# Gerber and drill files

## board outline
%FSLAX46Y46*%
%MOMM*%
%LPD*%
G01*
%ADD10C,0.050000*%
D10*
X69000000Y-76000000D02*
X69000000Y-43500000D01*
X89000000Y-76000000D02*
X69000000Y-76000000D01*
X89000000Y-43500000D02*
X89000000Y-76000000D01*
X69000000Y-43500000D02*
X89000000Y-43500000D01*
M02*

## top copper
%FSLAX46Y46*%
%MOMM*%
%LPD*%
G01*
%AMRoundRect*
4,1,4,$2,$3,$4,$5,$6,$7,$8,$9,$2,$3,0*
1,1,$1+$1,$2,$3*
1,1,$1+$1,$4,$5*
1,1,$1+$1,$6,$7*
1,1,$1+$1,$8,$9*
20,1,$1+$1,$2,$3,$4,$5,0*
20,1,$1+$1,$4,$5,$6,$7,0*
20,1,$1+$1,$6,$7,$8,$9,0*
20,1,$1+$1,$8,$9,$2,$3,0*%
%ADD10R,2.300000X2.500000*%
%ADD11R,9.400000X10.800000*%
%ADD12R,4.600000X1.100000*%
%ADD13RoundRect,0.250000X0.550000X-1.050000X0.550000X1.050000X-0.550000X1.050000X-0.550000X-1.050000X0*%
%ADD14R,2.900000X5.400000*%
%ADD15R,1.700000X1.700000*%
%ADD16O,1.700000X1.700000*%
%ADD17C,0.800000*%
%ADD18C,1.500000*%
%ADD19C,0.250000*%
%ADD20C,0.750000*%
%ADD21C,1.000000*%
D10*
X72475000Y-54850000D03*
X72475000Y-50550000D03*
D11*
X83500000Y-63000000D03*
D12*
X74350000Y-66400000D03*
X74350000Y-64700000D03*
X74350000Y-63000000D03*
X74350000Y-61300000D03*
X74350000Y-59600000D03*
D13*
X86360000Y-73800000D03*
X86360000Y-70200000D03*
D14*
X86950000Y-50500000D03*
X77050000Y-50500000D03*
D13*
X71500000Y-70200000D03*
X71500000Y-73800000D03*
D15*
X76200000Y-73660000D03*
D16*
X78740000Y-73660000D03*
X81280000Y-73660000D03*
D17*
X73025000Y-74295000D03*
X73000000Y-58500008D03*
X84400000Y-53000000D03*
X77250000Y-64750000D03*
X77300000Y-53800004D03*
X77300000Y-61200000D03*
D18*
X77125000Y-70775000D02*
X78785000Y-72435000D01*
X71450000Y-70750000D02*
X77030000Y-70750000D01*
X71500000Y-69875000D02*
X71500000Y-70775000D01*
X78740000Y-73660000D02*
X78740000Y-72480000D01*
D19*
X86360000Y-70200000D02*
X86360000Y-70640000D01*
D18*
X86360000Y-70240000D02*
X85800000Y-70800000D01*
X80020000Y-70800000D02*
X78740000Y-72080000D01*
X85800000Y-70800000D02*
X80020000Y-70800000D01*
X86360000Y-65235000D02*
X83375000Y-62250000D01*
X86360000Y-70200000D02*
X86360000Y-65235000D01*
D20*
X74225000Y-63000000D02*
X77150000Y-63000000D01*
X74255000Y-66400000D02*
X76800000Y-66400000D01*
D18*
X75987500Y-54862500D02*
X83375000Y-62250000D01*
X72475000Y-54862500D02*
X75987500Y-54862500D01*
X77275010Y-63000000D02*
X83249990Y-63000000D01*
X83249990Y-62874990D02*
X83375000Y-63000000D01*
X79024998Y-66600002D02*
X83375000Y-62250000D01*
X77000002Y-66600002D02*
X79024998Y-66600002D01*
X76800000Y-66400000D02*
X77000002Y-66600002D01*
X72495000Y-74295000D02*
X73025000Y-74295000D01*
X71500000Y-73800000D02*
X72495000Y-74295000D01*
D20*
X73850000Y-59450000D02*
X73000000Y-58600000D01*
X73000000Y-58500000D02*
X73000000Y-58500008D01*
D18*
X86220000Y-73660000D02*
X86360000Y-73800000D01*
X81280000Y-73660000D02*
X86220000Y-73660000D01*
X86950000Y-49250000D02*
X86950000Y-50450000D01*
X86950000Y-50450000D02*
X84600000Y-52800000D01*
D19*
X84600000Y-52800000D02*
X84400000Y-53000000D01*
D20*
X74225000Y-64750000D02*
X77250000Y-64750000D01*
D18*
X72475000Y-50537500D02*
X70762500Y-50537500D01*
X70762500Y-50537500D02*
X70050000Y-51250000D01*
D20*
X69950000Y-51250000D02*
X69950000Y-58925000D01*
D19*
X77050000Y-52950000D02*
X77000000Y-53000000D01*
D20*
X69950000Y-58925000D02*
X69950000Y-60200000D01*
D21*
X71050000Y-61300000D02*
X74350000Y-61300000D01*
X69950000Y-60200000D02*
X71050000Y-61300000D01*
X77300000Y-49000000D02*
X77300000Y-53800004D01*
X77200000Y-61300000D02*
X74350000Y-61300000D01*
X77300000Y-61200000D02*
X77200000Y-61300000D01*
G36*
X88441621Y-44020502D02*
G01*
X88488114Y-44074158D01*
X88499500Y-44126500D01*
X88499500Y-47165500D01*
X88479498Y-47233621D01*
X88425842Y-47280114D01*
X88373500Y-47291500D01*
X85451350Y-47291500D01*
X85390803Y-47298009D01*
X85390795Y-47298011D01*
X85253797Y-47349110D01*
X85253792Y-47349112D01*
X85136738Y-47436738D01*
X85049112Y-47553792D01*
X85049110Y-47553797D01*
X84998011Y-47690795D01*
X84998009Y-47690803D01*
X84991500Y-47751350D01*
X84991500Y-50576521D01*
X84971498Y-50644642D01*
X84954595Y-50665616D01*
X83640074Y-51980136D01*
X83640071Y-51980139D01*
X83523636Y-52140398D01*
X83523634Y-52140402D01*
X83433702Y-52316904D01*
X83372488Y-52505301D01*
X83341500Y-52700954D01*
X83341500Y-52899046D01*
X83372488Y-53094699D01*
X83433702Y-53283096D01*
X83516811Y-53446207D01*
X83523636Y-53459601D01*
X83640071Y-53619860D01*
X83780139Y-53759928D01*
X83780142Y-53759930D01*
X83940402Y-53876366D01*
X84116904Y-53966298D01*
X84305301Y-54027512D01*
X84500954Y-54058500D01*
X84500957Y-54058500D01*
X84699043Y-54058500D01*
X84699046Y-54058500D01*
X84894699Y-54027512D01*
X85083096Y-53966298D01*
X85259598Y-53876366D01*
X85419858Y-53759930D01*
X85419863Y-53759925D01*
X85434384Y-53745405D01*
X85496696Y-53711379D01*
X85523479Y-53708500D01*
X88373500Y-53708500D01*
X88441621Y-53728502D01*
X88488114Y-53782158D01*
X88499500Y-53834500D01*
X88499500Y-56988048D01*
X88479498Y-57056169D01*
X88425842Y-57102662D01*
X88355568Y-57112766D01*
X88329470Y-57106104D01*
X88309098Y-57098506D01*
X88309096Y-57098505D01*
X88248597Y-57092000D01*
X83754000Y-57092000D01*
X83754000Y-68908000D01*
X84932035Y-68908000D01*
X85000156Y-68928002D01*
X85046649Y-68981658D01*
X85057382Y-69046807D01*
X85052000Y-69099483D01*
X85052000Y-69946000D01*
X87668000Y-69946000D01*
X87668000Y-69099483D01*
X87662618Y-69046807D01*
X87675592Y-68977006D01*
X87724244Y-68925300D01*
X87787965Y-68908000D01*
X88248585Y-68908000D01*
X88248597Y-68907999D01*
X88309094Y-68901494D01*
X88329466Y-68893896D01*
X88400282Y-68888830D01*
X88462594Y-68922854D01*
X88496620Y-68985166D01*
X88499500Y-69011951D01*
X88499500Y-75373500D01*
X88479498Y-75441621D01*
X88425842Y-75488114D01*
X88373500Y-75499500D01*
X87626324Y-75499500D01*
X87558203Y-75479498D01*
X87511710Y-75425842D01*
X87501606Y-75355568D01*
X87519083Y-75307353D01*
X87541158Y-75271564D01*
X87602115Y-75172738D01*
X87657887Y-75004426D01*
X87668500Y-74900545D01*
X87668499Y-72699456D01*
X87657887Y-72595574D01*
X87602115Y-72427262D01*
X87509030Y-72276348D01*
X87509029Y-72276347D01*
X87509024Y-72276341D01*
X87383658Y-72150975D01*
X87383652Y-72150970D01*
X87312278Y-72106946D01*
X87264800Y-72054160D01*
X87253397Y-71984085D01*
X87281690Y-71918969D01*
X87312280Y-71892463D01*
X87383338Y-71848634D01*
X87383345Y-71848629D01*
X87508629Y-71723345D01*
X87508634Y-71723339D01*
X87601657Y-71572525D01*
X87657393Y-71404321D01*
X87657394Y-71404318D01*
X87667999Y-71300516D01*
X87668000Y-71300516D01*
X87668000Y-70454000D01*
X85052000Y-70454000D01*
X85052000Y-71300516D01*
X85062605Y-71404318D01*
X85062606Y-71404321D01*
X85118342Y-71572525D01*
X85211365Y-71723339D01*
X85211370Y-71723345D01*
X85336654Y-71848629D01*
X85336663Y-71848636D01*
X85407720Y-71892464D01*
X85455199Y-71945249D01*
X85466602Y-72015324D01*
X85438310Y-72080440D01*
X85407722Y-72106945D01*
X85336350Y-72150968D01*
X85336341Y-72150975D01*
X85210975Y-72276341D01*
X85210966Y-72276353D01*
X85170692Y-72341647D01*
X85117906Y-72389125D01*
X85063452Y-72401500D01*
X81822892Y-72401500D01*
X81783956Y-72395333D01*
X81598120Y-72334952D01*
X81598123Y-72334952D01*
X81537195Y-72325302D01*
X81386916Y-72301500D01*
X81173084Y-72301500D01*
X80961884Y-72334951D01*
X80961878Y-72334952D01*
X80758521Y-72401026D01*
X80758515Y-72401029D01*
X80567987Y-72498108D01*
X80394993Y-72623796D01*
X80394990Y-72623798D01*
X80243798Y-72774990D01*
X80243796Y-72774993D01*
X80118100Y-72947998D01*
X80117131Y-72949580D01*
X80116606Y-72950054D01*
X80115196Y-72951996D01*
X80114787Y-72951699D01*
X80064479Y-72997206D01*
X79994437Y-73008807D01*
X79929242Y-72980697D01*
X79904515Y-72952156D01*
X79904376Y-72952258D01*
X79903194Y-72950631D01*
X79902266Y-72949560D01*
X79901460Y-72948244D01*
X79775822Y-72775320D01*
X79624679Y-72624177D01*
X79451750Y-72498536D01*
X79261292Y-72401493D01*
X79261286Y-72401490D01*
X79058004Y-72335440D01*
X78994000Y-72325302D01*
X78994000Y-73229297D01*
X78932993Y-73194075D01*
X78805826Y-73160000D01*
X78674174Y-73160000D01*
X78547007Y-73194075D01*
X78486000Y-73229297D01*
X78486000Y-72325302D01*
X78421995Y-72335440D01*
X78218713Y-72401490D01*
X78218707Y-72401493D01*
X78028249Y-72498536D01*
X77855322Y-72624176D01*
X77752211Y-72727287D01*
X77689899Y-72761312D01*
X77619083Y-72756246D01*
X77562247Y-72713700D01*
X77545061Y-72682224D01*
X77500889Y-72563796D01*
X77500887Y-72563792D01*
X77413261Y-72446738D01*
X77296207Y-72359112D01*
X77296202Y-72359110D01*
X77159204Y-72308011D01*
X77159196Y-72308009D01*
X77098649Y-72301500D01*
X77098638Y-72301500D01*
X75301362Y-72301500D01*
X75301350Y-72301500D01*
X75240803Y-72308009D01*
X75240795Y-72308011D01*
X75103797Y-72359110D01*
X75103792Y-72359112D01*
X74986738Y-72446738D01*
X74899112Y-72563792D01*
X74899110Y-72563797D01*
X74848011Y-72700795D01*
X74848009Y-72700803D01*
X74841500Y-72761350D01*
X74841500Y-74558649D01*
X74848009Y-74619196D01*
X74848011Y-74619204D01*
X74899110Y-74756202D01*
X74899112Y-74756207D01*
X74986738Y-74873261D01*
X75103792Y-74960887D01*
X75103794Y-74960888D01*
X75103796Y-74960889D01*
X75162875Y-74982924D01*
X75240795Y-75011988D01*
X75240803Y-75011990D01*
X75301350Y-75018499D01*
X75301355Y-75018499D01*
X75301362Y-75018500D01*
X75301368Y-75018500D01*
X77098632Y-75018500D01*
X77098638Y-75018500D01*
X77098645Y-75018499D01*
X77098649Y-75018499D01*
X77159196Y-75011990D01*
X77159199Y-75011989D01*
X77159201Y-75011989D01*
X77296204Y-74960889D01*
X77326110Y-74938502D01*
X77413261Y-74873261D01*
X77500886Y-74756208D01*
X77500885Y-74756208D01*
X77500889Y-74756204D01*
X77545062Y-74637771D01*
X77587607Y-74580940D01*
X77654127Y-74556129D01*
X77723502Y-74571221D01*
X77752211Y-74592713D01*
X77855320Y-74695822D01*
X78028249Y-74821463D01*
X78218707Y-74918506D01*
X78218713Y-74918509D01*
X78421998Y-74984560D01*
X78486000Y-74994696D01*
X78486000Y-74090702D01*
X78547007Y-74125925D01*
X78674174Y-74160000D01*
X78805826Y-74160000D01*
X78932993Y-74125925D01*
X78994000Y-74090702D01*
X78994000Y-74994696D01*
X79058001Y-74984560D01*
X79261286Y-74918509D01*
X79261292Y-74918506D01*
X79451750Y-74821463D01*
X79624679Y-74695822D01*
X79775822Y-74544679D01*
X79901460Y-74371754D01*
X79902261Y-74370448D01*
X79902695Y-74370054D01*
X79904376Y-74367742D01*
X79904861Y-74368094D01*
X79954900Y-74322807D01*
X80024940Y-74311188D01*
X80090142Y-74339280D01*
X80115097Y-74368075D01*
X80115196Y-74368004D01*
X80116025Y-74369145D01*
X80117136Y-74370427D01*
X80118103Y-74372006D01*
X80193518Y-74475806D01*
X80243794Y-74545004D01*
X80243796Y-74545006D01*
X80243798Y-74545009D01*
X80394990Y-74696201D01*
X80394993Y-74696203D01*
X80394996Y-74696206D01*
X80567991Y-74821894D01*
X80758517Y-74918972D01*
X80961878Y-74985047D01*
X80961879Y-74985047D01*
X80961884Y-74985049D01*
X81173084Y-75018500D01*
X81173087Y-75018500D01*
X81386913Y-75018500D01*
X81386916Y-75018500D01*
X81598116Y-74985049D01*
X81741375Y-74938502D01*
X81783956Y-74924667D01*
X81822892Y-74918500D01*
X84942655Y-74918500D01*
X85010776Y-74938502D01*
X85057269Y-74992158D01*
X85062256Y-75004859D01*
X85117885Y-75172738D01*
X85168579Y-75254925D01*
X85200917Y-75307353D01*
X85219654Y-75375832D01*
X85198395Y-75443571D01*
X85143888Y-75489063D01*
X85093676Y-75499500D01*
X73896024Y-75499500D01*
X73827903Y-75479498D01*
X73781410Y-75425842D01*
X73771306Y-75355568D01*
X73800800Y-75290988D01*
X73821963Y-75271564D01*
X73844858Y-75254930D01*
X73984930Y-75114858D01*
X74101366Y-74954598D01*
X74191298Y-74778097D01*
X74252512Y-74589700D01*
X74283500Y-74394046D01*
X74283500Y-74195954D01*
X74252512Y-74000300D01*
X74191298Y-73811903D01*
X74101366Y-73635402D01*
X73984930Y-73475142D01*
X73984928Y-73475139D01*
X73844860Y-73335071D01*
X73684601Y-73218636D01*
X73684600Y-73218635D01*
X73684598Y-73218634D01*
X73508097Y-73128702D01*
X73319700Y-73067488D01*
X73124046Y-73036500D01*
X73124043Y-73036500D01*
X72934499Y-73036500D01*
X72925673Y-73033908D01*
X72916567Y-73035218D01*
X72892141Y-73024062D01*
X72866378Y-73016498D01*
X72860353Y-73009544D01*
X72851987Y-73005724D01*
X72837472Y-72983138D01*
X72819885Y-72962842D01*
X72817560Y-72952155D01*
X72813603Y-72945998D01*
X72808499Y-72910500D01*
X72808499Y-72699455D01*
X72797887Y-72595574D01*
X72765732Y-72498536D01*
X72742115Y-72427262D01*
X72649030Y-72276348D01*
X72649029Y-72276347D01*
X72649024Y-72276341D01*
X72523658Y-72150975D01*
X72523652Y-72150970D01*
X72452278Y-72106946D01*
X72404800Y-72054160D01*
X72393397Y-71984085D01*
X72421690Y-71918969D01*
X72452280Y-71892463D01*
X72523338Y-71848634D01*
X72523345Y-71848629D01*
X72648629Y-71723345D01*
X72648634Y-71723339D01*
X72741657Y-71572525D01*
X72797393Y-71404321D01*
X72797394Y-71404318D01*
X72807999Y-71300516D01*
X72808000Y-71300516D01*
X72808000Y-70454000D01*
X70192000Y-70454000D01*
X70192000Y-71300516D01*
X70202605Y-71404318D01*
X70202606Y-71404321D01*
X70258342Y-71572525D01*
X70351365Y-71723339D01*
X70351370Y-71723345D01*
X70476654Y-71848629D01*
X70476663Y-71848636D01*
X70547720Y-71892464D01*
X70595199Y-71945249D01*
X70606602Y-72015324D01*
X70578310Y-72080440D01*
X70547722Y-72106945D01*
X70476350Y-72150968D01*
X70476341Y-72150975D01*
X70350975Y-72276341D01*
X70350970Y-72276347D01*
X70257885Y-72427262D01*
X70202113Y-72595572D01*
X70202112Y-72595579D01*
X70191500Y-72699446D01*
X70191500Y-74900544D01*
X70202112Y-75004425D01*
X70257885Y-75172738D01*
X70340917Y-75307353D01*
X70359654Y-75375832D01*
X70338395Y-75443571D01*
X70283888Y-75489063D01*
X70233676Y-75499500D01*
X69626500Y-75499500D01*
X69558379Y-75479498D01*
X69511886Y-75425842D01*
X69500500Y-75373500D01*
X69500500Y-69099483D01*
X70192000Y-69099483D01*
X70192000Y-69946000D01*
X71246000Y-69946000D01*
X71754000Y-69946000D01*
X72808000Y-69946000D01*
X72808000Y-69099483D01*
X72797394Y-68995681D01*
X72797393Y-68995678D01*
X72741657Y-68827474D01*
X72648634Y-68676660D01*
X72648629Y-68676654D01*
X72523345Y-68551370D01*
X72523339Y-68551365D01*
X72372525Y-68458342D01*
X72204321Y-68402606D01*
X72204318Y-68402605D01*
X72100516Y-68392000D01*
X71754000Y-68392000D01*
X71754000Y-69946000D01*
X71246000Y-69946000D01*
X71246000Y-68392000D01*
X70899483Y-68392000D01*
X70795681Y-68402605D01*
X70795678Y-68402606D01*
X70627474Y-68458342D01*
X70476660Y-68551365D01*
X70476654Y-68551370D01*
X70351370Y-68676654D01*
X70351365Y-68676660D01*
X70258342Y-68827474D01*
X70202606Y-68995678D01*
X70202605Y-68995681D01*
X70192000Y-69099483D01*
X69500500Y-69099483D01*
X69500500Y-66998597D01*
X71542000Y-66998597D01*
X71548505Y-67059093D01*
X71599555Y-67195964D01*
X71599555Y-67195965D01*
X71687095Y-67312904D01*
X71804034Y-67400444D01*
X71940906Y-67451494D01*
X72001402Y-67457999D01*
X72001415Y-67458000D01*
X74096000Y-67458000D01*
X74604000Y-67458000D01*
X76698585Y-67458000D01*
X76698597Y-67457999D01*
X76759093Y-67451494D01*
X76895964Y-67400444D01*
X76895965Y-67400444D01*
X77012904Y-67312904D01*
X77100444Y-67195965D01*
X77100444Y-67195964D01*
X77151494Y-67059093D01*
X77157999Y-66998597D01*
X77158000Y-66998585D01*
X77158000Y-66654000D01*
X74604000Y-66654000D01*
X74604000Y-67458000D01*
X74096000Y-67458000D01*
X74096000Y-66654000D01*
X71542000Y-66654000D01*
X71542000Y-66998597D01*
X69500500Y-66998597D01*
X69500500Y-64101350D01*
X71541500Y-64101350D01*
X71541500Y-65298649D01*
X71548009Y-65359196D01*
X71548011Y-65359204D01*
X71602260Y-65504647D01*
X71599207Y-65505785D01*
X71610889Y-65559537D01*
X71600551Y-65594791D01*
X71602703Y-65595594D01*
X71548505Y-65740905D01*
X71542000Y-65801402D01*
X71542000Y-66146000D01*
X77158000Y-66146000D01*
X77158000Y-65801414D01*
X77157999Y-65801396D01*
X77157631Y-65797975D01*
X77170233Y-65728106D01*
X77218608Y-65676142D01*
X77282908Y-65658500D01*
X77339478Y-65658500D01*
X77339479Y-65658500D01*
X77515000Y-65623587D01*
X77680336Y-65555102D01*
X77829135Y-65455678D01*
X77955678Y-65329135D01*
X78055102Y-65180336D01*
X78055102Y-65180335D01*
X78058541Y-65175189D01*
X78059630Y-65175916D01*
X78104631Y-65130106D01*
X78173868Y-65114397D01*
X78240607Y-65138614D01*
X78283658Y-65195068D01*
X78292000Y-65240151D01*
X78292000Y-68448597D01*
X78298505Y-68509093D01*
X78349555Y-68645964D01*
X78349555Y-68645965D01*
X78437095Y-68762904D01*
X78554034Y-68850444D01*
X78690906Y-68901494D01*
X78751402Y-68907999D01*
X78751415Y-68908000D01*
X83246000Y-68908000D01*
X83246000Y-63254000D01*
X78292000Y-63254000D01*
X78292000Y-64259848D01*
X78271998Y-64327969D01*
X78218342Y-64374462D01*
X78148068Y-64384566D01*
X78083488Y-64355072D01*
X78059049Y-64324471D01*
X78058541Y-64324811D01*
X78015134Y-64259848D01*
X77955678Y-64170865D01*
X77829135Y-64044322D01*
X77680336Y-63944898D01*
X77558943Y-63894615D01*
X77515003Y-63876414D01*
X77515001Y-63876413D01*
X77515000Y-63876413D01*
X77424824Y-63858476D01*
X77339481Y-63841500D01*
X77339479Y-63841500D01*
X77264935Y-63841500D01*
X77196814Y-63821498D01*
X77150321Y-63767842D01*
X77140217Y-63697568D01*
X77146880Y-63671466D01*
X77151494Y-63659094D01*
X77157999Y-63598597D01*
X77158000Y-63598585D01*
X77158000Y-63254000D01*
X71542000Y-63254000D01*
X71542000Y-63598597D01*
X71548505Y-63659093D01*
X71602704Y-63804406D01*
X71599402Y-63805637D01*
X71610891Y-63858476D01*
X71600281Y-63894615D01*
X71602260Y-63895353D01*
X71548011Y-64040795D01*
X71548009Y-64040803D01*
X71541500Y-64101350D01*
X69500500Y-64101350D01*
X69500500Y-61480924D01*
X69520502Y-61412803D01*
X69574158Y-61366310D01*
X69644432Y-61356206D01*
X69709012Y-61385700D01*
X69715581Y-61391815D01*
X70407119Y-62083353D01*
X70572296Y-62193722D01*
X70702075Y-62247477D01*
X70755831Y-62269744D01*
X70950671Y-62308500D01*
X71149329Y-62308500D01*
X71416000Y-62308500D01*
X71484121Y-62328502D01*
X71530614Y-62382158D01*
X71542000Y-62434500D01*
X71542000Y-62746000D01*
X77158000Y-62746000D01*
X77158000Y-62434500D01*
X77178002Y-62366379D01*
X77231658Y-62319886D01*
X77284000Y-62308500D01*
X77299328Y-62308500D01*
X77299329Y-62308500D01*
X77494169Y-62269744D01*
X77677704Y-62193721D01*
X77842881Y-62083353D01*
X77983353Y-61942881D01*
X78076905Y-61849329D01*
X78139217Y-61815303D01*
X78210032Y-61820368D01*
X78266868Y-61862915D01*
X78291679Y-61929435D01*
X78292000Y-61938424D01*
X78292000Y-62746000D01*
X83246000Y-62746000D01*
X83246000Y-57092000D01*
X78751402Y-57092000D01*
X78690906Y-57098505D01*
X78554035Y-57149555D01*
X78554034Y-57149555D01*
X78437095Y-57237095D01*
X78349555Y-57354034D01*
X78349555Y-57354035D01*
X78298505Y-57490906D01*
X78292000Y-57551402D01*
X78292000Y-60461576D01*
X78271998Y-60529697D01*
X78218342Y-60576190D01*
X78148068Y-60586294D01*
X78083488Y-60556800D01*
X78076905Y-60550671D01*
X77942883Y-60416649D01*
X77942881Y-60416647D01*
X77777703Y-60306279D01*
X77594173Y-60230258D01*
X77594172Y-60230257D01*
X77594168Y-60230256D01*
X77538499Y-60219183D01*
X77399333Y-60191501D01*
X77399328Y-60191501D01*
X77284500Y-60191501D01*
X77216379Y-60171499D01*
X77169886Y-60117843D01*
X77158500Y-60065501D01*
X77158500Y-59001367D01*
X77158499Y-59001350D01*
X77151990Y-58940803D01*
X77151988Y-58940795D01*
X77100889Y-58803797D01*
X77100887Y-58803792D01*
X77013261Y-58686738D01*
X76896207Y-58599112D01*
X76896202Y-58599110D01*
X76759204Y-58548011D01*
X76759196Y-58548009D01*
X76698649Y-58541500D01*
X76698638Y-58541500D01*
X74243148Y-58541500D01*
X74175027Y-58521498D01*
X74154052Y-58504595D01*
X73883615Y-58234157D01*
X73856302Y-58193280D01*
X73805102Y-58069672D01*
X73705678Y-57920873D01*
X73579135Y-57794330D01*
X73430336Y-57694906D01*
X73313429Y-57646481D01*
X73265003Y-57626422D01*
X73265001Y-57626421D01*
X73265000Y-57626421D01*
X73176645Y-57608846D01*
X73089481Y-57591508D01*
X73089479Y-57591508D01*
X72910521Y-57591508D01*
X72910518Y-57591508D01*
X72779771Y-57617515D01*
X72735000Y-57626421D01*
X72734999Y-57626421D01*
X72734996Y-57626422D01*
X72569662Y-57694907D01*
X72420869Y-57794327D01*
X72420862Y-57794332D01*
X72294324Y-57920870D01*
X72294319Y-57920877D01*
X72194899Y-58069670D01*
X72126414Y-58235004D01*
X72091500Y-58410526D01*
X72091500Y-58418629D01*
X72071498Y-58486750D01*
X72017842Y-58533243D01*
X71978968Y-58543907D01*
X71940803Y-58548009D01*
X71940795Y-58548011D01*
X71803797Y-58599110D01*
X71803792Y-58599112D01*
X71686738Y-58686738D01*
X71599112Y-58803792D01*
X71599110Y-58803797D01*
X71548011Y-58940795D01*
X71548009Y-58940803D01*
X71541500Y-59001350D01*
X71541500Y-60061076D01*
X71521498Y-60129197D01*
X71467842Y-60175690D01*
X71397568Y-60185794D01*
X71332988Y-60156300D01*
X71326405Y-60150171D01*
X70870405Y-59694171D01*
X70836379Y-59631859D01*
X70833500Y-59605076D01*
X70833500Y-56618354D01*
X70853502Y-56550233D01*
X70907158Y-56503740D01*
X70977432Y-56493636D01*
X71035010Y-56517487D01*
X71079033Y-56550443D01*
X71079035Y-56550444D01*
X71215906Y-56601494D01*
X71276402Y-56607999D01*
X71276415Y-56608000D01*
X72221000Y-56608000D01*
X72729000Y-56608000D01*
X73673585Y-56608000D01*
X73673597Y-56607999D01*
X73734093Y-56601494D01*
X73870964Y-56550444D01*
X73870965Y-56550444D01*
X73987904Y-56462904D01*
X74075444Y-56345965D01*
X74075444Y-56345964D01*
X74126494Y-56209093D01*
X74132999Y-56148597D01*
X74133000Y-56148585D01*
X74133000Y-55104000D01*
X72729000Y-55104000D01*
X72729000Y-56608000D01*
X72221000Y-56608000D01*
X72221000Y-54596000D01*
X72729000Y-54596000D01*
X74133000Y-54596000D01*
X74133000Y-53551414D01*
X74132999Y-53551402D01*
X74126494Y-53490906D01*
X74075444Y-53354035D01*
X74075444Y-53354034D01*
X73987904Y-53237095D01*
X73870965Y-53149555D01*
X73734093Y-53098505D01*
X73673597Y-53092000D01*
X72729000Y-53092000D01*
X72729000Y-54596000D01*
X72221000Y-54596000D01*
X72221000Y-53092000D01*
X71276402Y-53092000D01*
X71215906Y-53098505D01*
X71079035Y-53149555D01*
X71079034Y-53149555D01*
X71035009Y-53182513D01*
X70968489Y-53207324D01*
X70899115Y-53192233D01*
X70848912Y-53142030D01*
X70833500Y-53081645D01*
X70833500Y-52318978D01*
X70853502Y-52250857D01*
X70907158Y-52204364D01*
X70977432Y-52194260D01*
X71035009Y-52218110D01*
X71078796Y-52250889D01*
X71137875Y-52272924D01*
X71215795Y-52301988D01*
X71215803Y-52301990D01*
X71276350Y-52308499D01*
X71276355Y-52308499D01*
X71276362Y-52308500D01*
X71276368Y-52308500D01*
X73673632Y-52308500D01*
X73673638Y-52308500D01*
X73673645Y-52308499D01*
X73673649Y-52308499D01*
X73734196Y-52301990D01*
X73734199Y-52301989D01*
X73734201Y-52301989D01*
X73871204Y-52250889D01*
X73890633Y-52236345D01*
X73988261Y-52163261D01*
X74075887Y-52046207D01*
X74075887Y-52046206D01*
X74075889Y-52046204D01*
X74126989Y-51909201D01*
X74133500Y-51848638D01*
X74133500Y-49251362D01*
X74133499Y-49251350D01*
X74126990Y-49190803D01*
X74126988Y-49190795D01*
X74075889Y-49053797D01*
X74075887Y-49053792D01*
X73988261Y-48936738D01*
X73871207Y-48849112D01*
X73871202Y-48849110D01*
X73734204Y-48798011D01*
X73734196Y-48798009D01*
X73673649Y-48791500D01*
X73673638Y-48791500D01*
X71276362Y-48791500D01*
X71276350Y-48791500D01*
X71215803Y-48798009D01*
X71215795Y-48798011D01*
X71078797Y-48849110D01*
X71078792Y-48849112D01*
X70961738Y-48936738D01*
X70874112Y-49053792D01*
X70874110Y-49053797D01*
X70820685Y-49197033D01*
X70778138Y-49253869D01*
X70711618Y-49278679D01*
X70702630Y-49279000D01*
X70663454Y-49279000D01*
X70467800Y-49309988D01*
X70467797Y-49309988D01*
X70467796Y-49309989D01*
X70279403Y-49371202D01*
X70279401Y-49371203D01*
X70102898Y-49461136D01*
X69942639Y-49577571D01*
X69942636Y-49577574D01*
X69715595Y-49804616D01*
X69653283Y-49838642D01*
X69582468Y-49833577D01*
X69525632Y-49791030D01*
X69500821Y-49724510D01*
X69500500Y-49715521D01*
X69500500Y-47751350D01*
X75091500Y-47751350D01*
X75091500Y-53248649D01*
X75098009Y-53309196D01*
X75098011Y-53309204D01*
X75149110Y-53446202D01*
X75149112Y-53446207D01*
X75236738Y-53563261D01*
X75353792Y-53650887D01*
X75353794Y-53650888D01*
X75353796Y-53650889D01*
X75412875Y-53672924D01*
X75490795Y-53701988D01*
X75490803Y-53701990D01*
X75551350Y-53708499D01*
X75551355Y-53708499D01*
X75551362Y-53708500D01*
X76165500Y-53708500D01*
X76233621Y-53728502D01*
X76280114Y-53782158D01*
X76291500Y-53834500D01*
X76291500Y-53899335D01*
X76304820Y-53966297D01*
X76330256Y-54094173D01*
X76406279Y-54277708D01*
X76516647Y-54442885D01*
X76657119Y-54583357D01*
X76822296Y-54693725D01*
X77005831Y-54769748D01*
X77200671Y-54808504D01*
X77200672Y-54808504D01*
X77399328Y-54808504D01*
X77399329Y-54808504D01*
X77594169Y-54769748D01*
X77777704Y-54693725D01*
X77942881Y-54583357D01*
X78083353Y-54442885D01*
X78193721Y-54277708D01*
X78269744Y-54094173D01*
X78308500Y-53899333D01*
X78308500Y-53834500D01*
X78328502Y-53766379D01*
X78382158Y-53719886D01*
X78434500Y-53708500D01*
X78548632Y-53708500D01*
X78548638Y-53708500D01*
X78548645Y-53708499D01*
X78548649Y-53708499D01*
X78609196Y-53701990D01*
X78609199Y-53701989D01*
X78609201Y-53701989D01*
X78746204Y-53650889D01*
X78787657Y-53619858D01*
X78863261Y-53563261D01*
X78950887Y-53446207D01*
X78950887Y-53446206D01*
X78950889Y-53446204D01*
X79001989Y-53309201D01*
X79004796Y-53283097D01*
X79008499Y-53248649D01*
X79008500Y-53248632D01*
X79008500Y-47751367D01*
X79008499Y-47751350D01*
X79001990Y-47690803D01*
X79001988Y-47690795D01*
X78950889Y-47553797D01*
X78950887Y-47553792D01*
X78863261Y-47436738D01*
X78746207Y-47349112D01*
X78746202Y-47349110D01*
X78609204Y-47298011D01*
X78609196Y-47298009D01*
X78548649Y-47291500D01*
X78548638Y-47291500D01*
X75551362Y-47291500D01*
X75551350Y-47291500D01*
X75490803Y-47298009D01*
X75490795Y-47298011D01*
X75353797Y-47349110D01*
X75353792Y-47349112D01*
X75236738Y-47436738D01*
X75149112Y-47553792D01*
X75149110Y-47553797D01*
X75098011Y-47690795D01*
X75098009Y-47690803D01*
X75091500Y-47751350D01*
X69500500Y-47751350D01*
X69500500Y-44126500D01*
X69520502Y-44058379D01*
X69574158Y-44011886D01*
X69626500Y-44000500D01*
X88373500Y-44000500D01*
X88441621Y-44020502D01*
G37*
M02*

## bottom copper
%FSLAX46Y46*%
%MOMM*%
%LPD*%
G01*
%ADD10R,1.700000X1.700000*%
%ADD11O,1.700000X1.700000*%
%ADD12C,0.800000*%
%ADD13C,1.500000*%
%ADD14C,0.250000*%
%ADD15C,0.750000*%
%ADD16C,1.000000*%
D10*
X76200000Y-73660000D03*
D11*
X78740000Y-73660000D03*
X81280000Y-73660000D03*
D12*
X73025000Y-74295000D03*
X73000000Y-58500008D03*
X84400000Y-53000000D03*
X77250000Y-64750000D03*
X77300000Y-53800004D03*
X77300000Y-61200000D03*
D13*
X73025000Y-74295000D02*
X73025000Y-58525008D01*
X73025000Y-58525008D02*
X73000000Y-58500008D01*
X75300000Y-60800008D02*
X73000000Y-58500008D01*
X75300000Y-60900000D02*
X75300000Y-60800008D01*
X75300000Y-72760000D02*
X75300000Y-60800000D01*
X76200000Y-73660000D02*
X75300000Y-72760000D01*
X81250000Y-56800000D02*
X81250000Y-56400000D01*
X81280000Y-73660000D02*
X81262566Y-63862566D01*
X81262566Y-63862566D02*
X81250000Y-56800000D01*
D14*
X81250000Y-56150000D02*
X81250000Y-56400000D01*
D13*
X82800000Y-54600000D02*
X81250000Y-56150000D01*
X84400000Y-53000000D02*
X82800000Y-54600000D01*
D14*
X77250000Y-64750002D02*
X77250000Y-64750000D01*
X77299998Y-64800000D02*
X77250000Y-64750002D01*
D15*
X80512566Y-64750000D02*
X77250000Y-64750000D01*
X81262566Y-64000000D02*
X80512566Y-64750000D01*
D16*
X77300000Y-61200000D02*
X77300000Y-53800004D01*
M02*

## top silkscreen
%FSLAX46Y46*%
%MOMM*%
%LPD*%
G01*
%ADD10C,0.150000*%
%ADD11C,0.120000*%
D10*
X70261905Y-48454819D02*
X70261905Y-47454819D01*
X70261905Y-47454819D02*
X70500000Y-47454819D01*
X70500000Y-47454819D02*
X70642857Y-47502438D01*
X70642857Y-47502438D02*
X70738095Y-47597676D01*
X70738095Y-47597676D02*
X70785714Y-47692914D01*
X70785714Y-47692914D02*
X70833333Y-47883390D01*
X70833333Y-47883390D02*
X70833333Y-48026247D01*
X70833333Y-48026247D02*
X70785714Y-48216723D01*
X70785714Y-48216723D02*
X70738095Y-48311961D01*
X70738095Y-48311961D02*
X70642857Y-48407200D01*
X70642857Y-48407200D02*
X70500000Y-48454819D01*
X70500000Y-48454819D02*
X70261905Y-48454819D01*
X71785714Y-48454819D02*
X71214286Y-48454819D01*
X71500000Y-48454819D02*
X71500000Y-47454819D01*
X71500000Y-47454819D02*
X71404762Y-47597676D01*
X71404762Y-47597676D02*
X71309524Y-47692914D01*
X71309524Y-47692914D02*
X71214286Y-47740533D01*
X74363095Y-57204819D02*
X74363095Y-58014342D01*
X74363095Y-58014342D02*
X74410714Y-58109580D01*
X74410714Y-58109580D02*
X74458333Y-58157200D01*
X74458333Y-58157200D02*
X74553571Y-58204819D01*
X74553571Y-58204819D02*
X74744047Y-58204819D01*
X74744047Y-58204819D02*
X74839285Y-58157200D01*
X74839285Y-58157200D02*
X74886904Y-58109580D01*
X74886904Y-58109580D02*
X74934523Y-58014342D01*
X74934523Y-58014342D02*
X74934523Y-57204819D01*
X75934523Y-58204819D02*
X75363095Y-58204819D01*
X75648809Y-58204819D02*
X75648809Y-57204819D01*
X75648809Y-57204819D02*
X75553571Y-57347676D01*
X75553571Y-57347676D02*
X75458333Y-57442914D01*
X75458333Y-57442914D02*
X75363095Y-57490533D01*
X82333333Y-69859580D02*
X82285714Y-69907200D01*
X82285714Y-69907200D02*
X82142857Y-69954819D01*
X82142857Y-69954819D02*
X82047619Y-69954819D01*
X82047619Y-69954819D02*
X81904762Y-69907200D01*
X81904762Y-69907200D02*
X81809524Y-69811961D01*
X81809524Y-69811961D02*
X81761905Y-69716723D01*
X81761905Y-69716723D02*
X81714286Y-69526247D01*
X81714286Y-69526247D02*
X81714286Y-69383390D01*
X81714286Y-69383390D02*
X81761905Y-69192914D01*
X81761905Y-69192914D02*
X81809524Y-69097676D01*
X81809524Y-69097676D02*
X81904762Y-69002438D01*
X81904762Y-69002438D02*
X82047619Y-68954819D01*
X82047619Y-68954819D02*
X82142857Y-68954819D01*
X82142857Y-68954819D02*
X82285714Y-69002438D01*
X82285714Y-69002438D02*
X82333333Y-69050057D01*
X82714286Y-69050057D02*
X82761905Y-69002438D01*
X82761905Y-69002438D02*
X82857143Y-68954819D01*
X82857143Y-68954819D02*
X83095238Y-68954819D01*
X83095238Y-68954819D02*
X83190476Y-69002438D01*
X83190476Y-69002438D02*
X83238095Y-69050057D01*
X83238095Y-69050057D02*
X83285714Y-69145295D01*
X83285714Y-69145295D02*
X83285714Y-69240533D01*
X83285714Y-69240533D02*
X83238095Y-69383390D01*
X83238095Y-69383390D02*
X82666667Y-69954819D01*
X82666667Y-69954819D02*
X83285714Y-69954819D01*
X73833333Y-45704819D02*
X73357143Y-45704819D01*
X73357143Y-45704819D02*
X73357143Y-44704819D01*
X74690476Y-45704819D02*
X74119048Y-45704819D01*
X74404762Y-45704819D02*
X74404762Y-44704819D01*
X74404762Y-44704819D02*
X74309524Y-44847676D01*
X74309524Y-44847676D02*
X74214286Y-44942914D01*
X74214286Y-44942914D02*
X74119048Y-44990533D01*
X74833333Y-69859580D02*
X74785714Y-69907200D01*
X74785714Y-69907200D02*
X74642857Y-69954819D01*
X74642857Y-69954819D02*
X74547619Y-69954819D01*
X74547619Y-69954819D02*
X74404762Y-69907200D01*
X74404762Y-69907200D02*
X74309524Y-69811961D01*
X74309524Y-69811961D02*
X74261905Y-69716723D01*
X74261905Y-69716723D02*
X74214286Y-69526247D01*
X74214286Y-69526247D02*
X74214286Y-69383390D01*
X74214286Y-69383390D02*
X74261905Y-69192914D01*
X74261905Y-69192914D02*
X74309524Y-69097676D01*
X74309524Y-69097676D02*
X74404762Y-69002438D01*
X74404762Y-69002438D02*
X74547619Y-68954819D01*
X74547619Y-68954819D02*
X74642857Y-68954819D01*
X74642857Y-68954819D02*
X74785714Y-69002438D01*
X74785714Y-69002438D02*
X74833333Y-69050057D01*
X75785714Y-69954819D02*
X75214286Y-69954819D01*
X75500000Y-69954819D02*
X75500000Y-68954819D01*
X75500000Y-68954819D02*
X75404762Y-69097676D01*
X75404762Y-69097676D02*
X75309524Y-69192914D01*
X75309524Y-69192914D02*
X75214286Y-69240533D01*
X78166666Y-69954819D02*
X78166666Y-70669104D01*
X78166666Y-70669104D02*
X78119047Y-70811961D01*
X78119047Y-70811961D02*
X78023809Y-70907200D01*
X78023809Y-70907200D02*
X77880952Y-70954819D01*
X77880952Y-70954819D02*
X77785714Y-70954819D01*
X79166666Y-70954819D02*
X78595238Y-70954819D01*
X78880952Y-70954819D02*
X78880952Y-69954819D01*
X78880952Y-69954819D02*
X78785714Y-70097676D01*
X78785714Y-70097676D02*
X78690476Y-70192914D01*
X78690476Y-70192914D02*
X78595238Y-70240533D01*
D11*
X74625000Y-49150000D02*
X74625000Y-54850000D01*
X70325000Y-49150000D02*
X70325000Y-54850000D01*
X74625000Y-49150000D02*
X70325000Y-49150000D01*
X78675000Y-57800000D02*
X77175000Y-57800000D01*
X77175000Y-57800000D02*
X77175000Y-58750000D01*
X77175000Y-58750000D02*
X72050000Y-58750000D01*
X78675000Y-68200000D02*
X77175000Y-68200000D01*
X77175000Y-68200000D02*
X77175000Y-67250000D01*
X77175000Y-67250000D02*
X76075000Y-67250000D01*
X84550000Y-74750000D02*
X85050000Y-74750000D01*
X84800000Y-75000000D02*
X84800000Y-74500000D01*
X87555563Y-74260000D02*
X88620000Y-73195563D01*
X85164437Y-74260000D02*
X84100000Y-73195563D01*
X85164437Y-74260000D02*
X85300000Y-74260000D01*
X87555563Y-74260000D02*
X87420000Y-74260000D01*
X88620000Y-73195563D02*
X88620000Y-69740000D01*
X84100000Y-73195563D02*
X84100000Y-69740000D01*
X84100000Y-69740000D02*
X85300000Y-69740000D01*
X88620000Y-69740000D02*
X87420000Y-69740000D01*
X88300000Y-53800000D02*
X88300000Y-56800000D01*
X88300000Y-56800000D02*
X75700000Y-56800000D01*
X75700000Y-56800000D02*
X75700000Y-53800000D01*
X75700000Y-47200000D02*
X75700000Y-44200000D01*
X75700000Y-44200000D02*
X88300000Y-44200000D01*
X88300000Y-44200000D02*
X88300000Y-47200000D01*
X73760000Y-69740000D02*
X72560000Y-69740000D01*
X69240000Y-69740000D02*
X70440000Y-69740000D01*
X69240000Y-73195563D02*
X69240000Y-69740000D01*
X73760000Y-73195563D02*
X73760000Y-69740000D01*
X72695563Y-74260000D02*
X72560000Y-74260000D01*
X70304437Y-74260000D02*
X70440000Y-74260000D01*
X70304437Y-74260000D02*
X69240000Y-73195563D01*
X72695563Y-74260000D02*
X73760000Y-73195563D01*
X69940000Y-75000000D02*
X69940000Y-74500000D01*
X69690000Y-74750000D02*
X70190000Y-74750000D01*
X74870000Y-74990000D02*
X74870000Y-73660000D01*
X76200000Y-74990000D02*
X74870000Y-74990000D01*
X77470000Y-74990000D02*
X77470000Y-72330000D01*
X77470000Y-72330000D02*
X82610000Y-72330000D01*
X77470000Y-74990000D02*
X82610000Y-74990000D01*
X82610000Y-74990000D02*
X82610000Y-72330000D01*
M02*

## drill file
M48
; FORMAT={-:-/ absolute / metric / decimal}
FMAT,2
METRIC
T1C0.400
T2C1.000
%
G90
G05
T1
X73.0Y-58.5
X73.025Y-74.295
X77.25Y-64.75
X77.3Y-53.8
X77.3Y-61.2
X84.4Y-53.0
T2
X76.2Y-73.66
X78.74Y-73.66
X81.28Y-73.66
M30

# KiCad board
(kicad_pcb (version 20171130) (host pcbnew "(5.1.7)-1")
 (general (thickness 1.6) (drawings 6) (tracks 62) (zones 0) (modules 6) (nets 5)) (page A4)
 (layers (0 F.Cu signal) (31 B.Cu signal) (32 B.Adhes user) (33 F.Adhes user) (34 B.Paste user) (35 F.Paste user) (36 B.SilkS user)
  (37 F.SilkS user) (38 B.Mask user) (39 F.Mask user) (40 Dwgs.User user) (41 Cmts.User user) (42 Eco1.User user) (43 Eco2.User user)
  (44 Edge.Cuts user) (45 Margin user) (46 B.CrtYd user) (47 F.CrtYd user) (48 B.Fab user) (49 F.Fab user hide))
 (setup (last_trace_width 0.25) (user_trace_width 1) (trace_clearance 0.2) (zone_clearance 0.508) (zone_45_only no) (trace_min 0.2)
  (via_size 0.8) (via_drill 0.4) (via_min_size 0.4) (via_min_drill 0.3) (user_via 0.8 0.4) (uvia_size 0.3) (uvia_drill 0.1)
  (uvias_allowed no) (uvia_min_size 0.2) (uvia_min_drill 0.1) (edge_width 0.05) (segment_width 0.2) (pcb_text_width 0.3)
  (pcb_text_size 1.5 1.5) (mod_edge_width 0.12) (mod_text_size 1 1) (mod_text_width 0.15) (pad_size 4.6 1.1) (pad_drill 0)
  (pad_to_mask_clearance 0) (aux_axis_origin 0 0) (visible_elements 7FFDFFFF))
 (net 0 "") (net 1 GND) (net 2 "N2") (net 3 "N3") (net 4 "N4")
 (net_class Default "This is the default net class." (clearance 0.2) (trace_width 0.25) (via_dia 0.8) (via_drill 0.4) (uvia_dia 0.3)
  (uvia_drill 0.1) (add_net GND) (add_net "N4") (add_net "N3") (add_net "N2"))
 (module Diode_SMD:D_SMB (layer F.Cu) (at 72.475 52.7 270)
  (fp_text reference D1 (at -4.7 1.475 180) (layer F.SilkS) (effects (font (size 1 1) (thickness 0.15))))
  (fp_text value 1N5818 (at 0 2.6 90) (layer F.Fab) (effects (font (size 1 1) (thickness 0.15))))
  (fp_line (start -3.55 -2.15) (end 2.15 -2.15) (layer F.SilkS) (width 0.12))
  (fp_line (start -3.55 2.15) (end 2.15 2.15) (layer F.SilkS) (width 0.12))
  (fp_line (start -3.55 -2.15) (end -3.55 2.15) (layer F.SilkS) (width 0.12))
  (pad 2 smd rect (at 2.15 0 270) (size 2.5 2.3) (layers F.Cu F.Paste F.Mask) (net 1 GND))
  (pad 1 smd rect (at -2.15 0 270) (size 2.5 2.3) (layers F.Cu F.Paste F.Mask) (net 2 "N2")))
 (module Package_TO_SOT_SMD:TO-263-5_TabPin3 (layer F.Cu) (at 80.125 63)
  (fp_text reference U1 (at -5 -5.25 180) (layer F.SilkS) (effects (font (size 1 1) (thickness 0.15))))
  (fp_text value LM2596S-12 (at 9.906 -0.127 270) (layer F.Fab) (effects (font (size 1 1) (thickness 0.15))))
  (fp_line (start -1.45 -5.2) (end -2.95 -5.2) (layer F.SilkS) (width 0.12))
  (fp_line (start -2.95 -5.2) (end -2.95 -4.25) (layer F.SilkS) (width 0.12))
  (fp_line (start -2.95 -4.25) (end -8.075 -4.25) (layer F.SilkS) (width 0.12))
  (fp_line (start -1.45 5.2) (end -2.95 5.2) (layer F.SilkS) (width 0.12))
  (fp_line (start -2.95 5.2) (end -2.95 4.25) (layer F.SilkS) (width 0.12))
  (fp_line (start -2.95 4.25) (end -4.05 4.25) (layer F.SilkS) (width 0.12))
  (pad "" smd rect (at 0.95 2.775) (size 4.55 5.25) (layers F.Paste))
  (pad "" smd rect (at 5.8 -2.775) (size 4.55 5.25) (layers F.Paste))
  (pad "" smd rect (at 0.95 -2.775) (size 4.55 5.25) (layers F.Paste))
  (pad "" smd rect (at 5.8 2.775) (size 4.55 5.25) (layers F.Paste))
  (pad 3 smd rect (at 3.375 0) (size 9.4 10.8) (layers F.Cu F.Mask) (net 1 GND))
  (pad 5 smd rect (at -5.775 3.4) (size 4.6 1.1) (layers F.Cu F.Paste F.Mask) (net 1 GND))
  (pad FEDBACK smd rect (at -5.775 1.7) (size 4.6 1.1) (layers F.Cu F.Paste F.Mask) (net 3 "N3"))
  (pad 3 smd rect (at -5.775 0) (size 4.6 1.1) (layers F.Cu F.Paste F.Mask) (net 1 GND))
  (pad OUTPUT smd rect (at -5.775 -1.7) (size 4.6 1.1) (layers F.Cu F.Paste F.Mask) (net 2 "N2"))
  (pad INPUT smd rect (at -5.775 -3.4) (size 4.6 1.1) (layers F.Cu F.Paste F.Mask) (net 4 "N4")))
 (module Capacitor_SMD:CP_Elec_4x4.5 (layer F.Cu) (at 86.36 72 90)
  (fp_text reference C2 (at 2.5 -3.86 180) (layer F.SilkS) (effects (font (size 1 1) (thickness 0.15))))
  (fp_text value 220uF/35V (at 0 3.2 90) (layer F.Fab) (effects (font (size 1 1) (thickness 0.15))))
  (fp_line (start -2.75 -1.81) (end -2.75 -1.31) (layer F.SilkS) (width 0.12))
  (fp_line (start -3 -1.56) (end -2.5 -1.56) (layer F.SilkS) (width 0.12))
  (fp_line (start -2.26 1.195563) (end -1.195563 2.26) (layer F.SilkS) (width 0.12))
  (fp_line (start -2.26 -1.195563) (end -1.195563 -2.26) (layer F.SilkS) (width 0.12))
  (fp_line (start -2.26 -1.195563) (end -2.26 -1.06) (layer F.SilkS) (width 0.12))
  (fp_line (start -2.26 1.195563) (end -2.26 1.06) (layer F.SilkS) (width 0.12))
  (fp_line (start -1.195563 2.26) (end 2.26 2.26) (layer F.SilkS) (width 0.12))
  (fp_line (start -1.195563 -2.26) (end 2.26 -2.26) (layer F.SilkS) (width 0.12))
  (fp_line (start 2.26 -2.26) (end 2.26 -1.06) (layer F.SilkS) (width 0.12))
  (fp_line (start 2.26 2.26) (end 2.26 1.06) (layer F.SilkS) (width 0.12))
  (pad 1 smd roundrect (at -1.8 0 90) (size 2.6 1.6) (layers F.Cu F.Paste F.Mask) (roundrect_rratio 0.15625) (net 3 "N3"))
  (pad 2 smd roundrect (at 1.8 0 90) (size 2.6 1.6) (layers F.Cu F.Paste F.Mask) (roundrect_rratio 0.15625) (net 1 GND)))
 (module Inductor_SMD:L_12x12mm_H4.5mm (layer F.Cu) (at 82 50.5)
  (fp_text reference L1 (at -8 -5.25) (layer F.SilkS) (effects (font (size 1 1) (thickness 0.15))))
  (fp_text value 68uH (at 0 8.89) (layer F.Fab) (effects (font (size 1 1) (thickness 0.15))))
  (fp_line (start 6.3 3.3) (end 6.3 6.3) (layer F.SilkS) (width 0.12))
  (fp_line (start 6.3 6.3) (end -6.3 6.3) (layer F.SilkS) (width 0.12))
  (fp_line (start -6.3 6.3) (end -6.3 3.3) (layer F.SilkS) (width 0.12))
  (fp_line (start -6.3 -3.3) (end -6.3 -6.3) (layer F.SilkS) (width 0.12))
  (fp_line (start -6.3 -6.3) (end 6.3 -6.3) (layer F.SilkS) (width 0.12))
  (fp_line (start 6.3 -6.3) (end 6.3 -3.3) (layer F.SilkS) (width 0.12))
  (pad 2 smd rect (at 4.95 0) (size 2.9 5.4) (layers F.Cu F.Paste F.Mask) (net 3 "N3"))
  (pad 1 smd rect (at -4.95 0) (size 2.9 5.4) (layers F.Cu F.Paste F.Mask) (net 2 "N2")))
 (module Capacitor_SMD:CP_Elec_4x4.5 (layer F.Cu) (at 71.5 72 90)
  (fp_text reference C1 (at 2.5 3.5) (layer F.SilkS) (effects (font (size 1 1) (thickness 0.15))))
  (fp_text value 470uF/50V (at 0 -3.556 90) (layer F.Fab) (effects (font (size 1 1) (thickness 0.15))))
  (fp_line (start 2.26 2.26) (end 2.26 1.06) (layer F.SilkS) (width 0.12))
  (fp_line (start 2.26 -2.26) (end 2.26 -1.06) (layer F.SilkS) (width 0.12))
  (fp_line (start -1.195563 -2.26) (end 2.26 -2.26) (layer F.SilkS) (width 0.12))
  (fp_line (start -1.195563 2.26) (end 2.26 2.26) (layer F.SilkS) (width 0.12))
  (fp_line (start -2.26 1.195563) (end -2.26 1.06) (layer F.SilkS) (width 0.12))
  (fp_line (start -2.26 -1.195563) (end -2.26 -1.06) (layer F.SilkS) (width 0.12))
  (fp_line (start -2.26 -1.195563) (end -1.195563 -2.26) (layer F.SilkS) (width 0.12))
  (fp_line (start -2.26 1.195563) (end -1.195563 2.26) (layer F.SilkS) (width 0.12))
  (fp_line (start -3 -1.56) (end -2.5 -1.56) (layer F.SilkS) (width 0.12))
  (fp_line (start -2.75 -1.81) (end -2.75 -1.31) (layer F.SilkS) (width 0.12))
  (pad 2 smd roundrect (at 1.8 0 90) (size 2.6 1.6) (layers F.Cu F.Paste F.Mask) (roundrect_rratio 0.15625) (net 1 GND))
  (pad 1 smd roundrect (at -1.8 0 90) (size 2.6 1.6) (layers F.Cu F.Paste F.Mask) (roundrect_rratio 0.15625) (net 4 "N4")))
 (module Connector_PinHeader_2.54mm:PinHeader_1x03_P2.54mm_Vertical (layer F.Cu) (at 76.2 73.66 90)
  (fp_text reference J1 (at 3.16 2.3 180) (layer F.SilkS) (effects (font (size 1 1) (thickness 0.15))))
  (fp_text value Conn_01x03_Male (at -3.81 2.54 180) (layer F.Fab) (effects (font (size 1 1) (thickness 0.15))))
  (fp_line (start -1.33 -1.33) (end 0 -1.33) (layer F.SilkS) (width 0.12))
  (fp_line (start -1.33 0) (end -1.33 -1.33) (layer F.SilkS) (width 0.12))
  (fp_line (start -1.33 1.27) (end 1.33 1.27) (layer F.SilkS) (width 0.12))
  (fp_line (start 1.33 1.27) (end 1.33 6.41) (layer F.SilkS) (width 0.12))
  (fp_line (start -1.33 1.27) (end -1.33 6.41) (layer F.SilkS) (width 0.12))
  (fp_line (start -1.33 6.41) (end 1.33 6.41) (layer F.SilkS) (width 0.12))
  (pad 1 thru_hole rect (at 0 0 90) (size 1.7 1.7) (drill 1) (layers *.Cu *.Mask) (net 4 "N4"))
  (pad 2 thru_hole oval (at 0 2.54 90) (size 1.7 1.7) (drill 1) (layers *.Cu *.Mask) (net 1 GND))
  (pad 3 thru_hole oval (at 0 5.08 90) (size 1.7 1.7) (drill 1) (layers *.Cu *.Mask) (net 3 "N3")))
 (gr_line (start 69 76) (end 69 43.5) (layer Edge.Cuts) (width 0.05))
 (gr_line (start 89 76) (end 69 76) (layer Edge.Cuts) (width 0.05))
 (gr_line (start 89 43.5) (end 89 76) (layer Edge.Cuts) (width 0.05))
 (gr_line (start 69 43.5) (end 89 43.5) (layer Edge.Cuts) (width 0.05))
 (segment (start 77.125 70.775) (end 78.785 72.435) (width 1.5) (layer F.Cu) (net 1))
 (segment (start 71.45 70.75) (end 77.03 70.75) (width 1.5) (layer F.Cu) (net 1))
 (segment (start 71.5 69.875) (end 71.5 70.775) (width 1.5) (layer F.Cu) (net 1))
 (segment (start 78.74 73.66) (end 78.74 72.48) (width 1.5) (layer F.Cu) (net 1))
 (segment (start 86.36 70.2) (end 86.36 70.64) (width 0.25) (layer F.Cu) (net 1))
 (segment (start 86.36 70.24) (end 85.8 70.8) (width 1.5) (layer F.Cu) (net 1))
 (segment (start 80.02 70.8) (end 78.74 72.08) (width 1.5) (layer F.Cu) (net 1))
 (segment (start 85.8 70.8) (end 80.02 70.8) (width 1.5) (layer F.Cu) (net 1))
 (segment (start 86.36 65.235) (end 83.375 62.25) (width 1.5) (layer F.Cu) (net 1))
 (segment (start 86.36 70.2) (end 86.36 65.235) (width 1.5) (layer F.Cu) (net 1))
 (segment (start 74.225 63) (end 77.15 63) (width 0.75) (layer F.Cu) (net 1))
 (segment (start 74.255 66.4) (end 76.8 66.4) (width 0.75) (layer F.Cu) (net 1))
 (segment (start 75.9875 54.8625) (end 83.375 62.25) (width 1.5) (layer F.Cu) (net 1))
 (segment (start 72.475 54.8625) (end 75.9875 54.8625) (width 1.5) (layer F.Cu) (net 1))
 (segment (start 77.27501 63) (end 83.24999 63) (width 1.5) (layer F.Cu) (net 1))
 (segment (start 83.24999 62.87499) (end 83.375 63) (width 1.5) (layer F.Cu) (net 1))
 (segment (start 79.024998 66.600002) (end 83.375 62.25) (width 1.5) (layer F.Cu) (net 1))
 (segment (start 77.000002 66.600002) (end 79.024998 66.600002) (width 1.5) (layer F.Cu) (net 1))
 (segment (start 76.8 66.4) (end 77.000002 66.600002) (width 1.5) (layer F.Cu) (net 1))
 (via (at 73.025 74.295) (size 0.8) (drill 0.4) (layers F.Cu B.Cu) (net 4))
 (segment (start 72.495 74.295) (end 73.025 74.295) (width 1.5) (layer F.Cu) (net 4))
 (segment (start 71.5 73.8) (end 72.495 74.295) (width 1.5) (layer F.Cu) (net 4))
 (segment (start 73.85 59.45) (end 73 58.6) (width 0.75) (layer F.Cu) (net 4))
 (via (at 73 58.500008) (size 0.8) (drill 0.4) (layers F.Cu B.Cu) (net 4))
 (segment (start 73 58.5) (end 73 58.500008) (width 0.75) (layer F.Cu) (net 4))
 (segment (start 73.025 74.295) (end 73.025 58.525008) (width 1.5) (layer B.Cu) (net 4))
 (segment (start 73.025 58.525008) (end 73 58.500008) (width 1.5) (layer B.Cu) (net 4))
 (segment (start 75.3 60.800008) (end 73 58.500008) (width 1.5) (layer B.Cu) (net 4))
 (segment (start 75.3 60.9) (end 75.3 60.800008) (width 1.5) (layer B.Cu) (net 4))
 (segment (start 75.3 72.76) (end 75.3 60.8) (width 1.5) (layer B.Cu) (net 4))
 (segment (start 76.2 73.66) (end 75.3 72.76) (width 1.5) (layer B.Cu) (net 4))
 (segment (start 86.22 73.66) (end 86.36 73.8) (width 1.5) (layer F.Cu) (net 3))
 (segment (start 81.28 73.66) (end 86.22 73.66) (width 1.5) (layer F.Cu) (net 3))
 (segment (start 81.25 56.8) (end 81.25 56.4) (width 1.5) (layer B.Cu) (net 3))
 (segment (start 81.28 73.66) (end 81.262566 63.862566) (width 1.5) (layer B.Cu) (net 3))
 (segment (start 81.262566 63.862566) (end 81.25 56.8) (width 1.5) (layer B.Cu) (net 3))
 (segment (start 86.95 49.25) (end 86.95 50.45) (width 1.5) (layer F.Cu) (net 3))
 (segment (start 86.95 50.45) (end 84.6 52.8) (width 1.5) (layer F.Cu) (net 3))
 (via (at 84.4 53) (size 0.8) (drill 0.4) (layers F.Cu B.Cu) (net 3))
 (segment (start 84.6 52.8) (end 84.4 53) (width 0.25) (layer F.Cu) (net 3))
 (segment (start 81.25 56.15) (end 81.25 56.4) (width 0.25) (layer B.Cu) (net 3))
 (segment (start 82.8 54.6) (end 81.25 56.15) (width 1.5) (layer B.Cu) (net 3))
 (segment (start 84.4 53) (end 82.8 54.6) (width 1.5) (layer B.Cu) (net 3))
 (segment (start 77.25 64.750002) (end 77.25 64.75) (width 0.25) (layer B.Cu) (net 3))
 (segment (start 77.299998 64.8) (end 77.25 64.750002) (width 0.25) (layer B.Cu) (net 3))
 (segment (start 80.512566 64.75) (end 77.25 64.75) (width 0.75) (layer B.Cu) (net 3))
 (segment (start 81.262566 64) (end 80.512566 64.75) (width 0.75) (layer B.Cu) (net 3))
 (segment (start 74.225 64.75) (end 77.25 64.75) (width 0.75) (layer F.Cu) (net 3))
 (via (at 77.25 64.75) (size 0.8) (drill 0.4) (layers F.Cu B.Cu) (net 3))
 (segment (start 72.475 50.5375) (end 70.7625 50.5375) (width 1.5) (layer F.Cu) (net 2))
 (segment (start 70.7625 50.5375) (end 70.05 51.25) (width 1.5) (layer F.Cu) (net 2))
 (segment (start 69.95 51.25) (end 69.95 58.925) (width 0.75) (layer F.Cu) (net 2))
 (segment (start 77.05 52.95) (end 77 53) (width 0.25) (layer F.Cu) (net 2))
 (segment (start 69.95 58.925) (end 69.95 60.2) (width 0.75) (layer F.Cu) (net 2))
 (segment (start 71.05 61.3) (end 74.35 61.3) (width 1) (layer F.Cu) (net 2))
 (segment (start 69.95 60.2) (end 71.05 61.3) (width 1) (layer F.Cu) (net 2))
 (via (at 77.3 53.800004) (size 0.8) (drill 0.4) (layers F.Cu B.Cu) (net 2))
 (segment (start 77.3 49) (end 77.3 53.800004) (width 1) (layer F.Cu) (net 2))
 (via (at 77.3 61.2) (size 0.8) (drill 0.4) (layers F.Cu B.Cu) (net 2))
 (segment (start 77.2 61.3) (end 74.35 61.3) (width 1) (layer F.Cu) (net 2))
 (segment (start 77.3 61.2) (end 77.2 61.3) (width 1) (layer F.Cu) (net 2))
 (segment (start 77.3 61.2) (end 77.3 53.800004) (width 1) (layer B.Cu) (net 2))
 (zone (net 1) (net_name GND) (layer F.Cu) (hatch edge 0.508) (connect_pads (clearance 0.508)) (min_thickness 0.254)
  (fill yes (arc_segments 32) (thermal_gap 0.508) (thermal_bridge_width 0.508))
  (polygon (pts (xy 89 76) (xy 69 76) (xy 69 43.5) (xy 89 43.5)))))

